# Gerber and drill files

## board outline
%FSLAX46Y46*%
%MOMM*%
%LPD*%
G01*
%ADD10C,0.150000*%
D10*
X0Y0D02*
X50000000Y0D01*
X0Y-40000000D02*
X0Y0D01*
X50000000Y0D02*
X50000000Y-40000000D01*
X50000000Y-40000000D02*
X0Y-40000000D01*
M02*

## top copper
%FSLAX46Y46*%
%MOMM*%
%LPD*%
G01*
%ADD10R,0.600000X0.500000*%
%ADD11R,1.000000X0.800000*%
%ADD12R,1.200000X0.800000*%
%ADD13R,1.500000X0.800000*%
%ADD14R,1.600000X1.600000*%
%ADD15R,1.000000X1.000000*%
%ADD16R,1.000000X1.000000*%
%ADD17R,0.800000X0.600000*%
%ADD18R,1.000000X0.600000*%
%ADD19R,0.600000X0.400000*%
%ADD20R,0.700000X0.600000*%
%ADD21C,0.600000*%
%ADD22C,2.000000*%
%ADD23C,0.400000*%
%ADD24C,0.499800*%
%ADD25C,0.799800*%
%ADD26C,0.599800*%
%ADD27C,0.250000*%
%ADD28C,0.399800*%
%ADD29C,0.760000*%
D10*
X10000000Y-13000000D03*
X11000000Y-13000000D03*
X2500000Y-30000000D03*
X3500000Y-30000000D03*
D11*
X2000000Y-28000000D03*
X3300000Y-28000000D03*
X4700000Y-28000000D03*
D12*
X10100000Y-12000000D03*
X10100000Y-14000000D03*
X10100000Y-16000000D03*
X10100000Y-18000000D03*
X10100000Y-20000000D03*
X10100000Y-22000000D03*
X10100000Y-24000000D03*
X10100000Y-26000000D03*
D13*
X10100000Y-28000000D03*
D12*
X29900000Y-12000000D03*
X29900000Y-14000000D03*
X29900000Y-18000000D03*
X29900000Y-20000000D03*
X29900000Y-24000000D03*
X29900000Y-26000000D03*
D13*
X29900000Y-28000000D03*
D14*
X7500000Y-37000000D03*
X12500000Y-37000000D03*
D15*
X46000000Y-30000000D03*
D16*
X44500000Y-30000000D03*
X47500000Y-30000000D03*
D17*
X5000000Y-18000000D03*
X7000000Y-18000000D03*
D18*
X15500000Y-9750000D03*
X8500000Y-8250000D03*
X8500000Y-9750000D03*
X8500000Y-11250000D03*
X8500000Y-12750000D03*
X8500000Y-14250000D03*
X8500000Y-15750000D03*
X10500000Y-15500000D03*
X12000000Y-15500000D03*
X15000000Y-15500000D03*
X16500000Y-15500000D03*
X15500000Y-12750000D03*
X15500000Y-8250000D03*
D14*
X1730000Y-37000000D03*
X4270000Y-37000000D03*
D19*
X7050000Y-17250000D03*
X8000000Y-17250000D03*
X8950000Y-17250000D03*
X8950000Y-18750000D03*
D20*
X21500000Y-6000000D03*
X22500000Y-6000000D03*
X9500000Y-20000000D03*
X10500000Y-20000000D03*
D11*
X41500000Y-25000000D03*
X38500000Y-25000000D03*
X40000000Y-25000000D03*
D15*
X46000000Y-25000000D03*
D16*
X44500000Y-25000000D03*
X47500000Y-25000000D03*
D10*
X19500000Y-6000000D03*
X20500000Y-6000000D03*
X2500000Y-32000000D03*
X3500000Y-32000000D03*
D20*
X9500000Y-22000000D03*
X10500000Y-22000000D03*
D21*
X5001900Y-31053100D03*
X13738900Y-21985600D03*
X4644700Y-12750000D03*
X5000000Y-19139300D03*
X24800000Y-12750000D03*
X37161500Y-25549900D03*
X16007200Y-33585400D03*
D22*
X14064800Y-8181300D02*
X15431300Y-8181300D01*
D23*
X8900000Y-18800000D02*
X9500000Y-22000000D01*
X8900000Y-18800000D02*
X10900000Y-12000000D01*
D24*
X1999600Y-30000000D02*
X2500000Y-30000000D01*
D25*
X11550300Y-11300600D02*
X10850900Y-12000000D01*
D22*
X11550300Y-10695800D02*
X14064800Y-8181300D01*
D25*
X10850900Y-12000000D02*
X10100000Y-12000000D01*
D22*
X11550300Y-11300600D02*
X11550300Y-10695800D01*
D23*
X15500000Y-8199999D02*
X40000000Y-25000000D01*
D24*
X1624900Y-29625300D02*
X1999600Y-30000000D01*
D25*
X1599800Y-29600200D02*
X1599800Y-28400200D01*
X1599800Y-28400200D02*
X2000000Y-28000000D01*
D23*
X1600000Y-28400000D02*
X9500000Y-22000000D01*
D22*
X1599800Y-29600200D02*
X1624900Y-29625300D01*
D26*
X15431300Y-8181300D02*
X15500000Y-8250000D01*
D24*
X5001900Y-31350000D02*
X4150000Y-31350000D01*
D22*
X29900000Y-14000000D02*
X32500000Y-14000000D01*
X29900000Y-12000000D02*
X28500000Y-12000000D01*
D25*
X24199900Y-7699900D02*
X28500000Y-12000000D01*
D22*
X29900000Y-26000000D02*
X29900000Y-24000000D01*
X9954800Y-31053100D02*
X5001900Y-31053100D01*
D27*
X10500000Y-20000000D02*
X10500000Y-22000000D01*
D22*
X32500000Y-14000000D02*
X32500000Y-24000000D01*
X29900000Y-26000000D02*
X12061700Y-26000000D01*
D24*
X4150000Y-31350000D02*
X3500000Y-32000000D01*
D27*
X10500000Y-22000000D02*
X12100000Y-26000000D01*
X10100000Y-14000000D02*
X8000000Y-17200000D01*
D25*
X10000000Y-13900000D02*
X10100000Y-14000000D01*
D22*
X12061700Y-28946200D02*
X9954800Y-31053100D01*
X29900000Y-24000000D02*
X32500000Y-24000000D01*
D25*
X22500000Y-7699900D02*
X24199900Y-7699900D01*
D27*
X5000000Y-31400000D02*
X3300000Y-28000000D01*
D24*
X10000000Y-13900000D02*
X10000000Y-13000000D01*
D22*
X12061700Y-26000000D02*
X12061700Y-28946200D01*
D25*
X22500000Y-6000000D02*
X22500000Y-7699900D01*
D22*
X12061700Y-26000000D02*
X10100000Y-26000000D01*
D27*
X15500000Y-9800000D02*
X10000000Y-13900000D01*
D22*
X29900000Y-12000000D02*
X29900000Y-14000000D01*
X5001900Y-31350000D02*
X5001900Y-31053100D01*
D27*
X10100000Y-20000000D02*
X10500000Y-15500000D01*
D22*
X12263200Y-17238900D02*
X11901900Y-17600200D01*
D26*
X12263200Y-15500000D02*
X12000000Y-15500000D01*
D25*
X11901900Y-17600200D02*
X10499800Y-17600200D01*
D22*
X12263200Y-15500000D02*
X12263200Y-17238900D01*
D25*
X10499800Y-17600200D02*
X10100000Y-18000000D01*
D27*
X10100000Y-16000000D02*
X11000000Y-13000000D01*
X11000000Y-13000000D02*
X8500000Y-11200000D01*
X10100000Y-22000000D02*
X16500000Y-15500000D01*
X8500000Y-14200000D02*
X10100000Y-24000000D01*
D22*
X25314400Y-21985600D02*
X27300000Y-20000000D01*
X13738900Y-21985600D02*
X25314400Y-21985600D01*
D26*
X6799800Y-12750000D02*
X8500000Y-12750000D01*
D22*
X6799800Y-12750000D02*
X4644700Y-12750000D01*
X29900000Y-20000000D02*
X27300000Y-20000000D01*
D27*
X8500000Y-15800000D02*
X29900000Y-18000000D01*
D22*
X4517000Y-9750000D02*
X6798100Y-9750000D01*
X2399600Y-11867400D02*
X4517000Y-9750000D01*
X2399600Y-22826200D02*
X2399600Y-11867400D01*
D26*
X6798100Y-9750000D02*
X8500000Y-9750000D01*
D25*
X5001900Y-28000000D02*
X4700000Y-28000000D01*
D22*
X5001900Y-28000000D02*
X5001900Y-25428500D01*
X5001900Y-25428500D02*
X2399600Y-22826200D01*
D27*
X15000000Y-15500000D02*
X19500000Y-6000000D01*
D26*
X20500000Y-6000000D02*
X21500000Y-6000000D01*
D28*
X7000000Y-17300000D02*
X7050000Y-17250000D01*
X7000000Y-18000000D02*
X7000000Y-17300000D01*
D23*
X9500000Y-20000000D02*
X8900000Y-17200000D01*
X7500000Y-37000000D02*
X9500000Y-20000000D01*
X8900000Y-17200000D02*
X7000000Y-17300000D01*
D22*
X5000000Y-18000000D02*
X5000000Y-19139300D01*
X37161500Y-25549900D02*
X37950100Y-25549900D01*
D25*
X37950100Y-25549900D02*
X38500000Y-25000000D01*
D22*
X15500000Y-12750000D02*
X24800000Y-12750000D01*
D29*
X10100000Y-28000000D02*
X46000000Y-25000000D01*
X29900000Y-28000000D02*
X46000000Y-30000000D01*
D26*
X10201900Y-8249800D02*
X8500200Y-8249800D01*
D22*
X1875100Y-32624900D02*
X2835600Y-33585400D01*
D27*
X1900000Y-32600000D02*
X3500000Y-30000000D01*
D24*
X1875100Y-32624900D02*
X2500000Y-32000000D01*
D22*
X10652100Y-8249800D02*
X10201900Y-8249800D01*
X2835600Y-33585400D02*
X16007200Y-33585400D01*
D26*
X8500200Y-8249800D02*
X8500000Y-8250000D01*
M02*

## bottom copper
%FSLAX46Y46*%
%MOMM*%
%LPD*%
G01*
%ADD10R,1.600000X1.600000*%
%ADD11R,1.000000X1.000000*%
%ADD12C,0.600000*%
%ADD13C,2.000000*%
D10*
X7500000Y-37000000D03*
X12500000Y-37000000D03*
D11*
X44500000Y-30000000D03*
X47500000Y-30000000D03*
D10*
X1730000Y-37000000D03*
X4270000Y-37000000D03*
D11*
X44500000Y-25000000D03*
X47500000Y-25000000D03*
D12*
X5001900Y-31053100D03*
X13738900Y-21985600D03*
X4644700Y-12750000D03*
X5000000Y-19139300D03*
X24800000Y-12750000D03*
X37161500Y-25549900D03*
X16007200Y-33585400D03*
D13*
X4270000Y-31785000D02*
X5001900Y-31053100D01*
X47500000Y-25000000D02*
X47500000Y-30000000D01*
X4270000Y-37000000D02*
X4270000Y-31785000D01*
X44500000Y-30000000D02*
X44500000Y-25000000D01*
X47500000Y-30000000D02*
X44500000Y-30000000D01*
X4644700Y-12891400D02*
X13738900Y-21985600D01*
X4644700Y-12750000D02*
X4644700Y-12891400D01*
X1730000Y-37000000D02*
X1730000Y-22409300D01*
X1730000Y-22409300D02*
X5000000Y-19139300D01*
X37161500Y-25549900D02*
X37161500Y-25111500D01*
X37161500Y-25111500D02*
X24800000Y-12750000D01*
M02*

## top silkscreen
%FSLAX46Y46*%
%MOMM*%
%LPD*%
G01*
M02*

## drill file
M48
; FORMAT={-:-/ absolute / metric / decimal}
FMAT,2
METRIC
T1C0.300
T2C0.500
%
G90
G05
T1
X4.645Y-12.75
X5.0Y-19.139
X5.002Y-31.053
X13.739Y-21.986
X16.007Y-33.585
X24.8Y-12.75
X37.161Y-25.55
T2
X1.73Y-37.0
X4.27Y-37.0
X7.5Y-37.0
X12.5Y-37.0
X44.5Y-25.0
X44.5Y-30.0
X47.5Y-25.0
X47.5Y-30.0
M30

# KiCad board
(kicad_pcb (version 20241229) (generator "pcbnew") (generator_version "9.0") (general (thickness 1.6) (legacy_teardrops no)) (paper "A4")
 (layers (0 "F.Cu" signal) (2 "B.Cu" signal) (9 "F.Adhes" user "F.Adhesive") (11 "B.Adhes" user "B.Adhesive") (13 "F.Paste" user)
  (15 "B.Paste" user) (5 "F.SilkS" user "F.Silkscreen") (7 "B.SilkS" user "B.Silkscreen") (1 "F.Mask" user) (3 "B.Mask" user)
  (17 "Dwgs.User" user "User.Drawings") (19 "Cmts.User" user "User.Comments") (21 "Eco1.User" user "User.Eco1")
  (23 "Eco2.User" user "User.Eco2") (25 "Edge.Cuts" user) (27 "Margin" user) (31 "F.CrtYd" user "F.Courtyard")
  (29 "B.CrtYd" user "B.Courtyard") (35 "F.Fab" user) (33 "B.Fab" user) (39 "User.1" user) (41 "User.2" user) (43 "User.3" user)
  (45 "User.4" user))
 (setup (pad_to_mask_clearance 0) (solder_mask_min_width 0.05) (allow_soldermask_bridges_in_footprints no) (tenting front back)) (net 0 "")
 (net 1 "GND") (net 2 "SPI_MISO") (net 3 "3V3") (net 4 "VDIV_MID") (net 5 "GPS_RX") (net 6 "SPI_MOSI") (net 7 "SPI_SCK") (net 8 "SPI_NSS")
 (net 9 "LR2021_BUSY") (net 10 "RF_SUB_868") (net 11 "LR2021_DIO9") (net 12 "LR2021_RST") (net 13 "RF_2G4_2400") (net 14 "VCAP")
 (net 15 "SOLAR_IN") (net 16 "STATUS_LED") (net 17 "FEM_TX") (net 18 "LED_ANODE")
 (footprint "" (layer "F.Cu") (at 10.5 13)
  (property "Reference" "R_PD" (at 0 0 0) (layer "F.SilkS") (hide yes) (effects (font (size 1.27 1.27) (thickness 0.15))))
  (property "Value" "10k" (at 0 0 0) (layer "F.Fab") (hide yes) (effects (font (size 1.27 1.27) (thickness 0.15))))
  (pad "1" smd rect (at -0.5 0) (size 0.6 0.5) (layers "F.Cu" "F.Mask") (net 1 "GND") (thermal_bridge_angle 45))
  (pad "2" smd rect (at 0.5 0) (size 0.6 0.5) (layers "F.Cu" "F.Mask") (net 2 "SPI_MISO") (thermal_bridge_angle 45)))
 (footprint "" (layer "F.Cu") (at 3 30)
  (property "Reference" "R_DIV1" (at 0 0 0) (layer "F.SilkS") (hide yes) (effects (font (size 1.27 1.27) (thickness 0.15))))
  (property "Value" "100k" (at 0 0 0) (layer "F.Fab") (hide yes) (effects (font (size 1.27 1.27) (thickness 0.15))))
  (pad "1" smd rect (at -0.5 0) (size 0.6 0.5) (layers "F.Cu" "F.Mask") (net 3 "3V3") (thermal_bridge_angle 45))
  (pad "2" smd rect (at 0.5 0) (size 0.6 0.5) (layers "F.Cu" "F.Mask") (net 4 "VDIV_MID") (thermal_bridge_angle 45)))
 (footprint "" (layer "F.Cu") (at 4 28)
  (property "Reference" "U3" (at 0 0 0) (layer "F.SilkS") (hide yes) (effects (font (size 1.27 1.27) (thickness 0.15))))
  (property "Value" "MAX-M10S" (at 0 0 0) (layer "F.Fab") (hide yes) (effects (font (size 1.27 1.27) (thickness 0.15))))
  (pad "1" smd rect (at -2 0) (size 1 0.8) (layers "F.Cu" "F.Mask") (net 3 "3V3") (thermal_bridge_angle 45))
  (pad "2" smd rect (at -0.7 0) (size 1 0.8) (layers "F.Cu" "F.Mask") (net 1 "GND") (thermal_bridge_angle 45))
  (pad "3" smd rect (at 0.7 0) (size 1 0.8) (layers "F.Cu" "F.Mask") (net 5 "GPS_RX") (thermal_bridge_angle 45)))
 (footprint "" (layer "F.Cu") (at 20 20)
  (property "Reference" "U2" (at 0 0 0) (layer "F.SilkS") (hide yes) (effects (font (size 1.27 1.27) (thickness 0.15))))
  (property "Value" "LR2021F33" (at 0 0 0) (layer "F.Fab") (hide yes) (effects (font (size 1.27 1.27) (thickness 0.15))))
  (pad "1" smd rect (at -9.9 -8) (size 1.2 0.8) (layers "F.Cu" "F.Mask") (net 3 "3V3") (thermal_bridge_angle 45))
  (pad "2" smd rect (at -9.9 -6) (size 1.2 0.8) (layers "F.Cu" "F.Mask") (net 1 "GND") (thermal_bridge_angle 45))
  (pad "3" smd rect (at -9.9 -4) (size 1.2 0.8) (layers "F.Cu" "F.Mask") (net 2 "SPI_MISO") (thermal_bridge_angle 45))
  (pad "4" smd rect (at -9.9 -2) (size 1.2 0.8) (layers "F.Cu" "F.Mask") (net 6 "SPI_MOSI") (thermal_bridge_angle 45))
  (pad "5" smd rect (at -9.9 0) (size 1.2 0.8) (layers "F.Cu" "F.Mask") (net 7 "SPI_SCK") (thermal_bridge_angle 45))
  (pad "6" smd rect (at -9.9 2) (size 1.2 0.8) (layers "F.Cu" "F.Mask") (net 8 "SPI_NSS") (thermal_bridge_angle 45))
  (pad "7" smd rect (at -9.9 4) (size 1.2 0.8) (layers "F.Cu" "F.Mask") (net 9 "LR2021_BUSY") (thermal_bridge_angle 45))
  (pad "8" smd rect (at -9.9 6) (size 1.2 0.8) (layers "F.Cu" "F.Mask") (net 1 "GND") (thermal_bridge_angle 45))
  (pad "9" smd rect (at -9.9 8) (size 1.5 0.8) (layers "F.Cu" "F.Mask") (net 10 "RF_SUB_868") (thermal_bridge_angle 45))
  (pad "10" smd rect (at 9.9 -8) (size 1.2 0.8) (layers "F.Cu" "F.Mask") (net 1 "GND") (thermal_bridge_angle 45))
  (pad "11" smd rect (at 9.9 -6) (size 1.2 0.8) (layers "F.Cu" "F.Mask") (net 1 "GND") (thermal_bridge_angle 45))
  (pad "13" smd rect (at 9.9 -2) (size 1.2 0.8) (layers "F.Cu" "F.Mask") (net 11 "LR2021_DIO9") (thermal_bridge_angle 45))
  (pad "14" smd rect (at 9.9 0) (size 1.2 0.8) (layers "F.Cu" "F.Mask") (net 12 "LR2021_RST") (thermal_bridge_angle 45))
  (pad "16" smd rect (at 9.9 4) (size 1.2 0.8) (layers "F.Cu" "F.Mask") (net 1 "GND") (thermal_bridge_angle 45))
  (pad "17" smd rect (at 9.9 6) (size 1.2 0.8) (layers "F.Cu" "F.Mask") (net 1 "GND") (thermal_bridge_angle 45))
  (pad "18" smd rect (at 9.9 8) (size 1.5 0.8) (layers "F.Cu" "F.Mask") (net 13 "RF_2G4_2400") (thermal_bridge_angle 45)))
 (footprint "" (layer "F.Cu") (at 10 37)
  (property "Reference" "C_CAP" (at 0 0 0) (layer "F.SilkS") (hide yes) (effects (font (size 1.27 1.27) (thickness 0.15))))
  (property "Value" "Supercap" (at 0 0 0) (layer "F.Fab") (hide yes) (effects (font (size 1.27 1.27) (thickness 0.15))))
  (pad "1" thru_hole rect (at -2.5 0) (size 1.6 1.6) (drill 0.5) (layers "*.Cu" "*.Mask") (remove_unused_layers no) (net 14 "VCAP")
   (thermal_bridge_angle 45))
  (pad "2" thru_hole rect (at 2.5 0) (size 1.6 1.6) (drill 0.5) (layers "*.Cu" "*.Mask") (remove_unused_layers no) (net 1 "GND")
   (thermal_bridge_angle 45)))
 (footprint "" (layer "F.Cu") (at 46 30)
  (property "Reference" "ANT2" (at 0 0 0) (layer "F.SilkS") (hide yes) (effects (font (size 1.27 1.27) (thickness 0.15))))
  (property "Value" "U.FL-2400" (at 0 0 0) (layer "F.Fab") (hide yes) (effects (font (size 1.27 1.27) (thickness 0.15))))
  (pad "1" smd rect (at 0 0) (size 1 1) (layers "F.Cu" "F.Mask") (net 13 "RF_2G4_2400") (thermal_bridge_angle 45))
  (pad "2" thru_hole rect (at -1.5 0) (size 1 1) (drill 0.5) (layers "*.Cu" "*.Mask") (remove_unused_layers no) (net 1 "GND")
   (thermal_bridge_angle 45))
  (pad "3" thru_hole rect (at 1.5 0) (size 1 1) (drill 0.5) (layers "*.Cu" "*.Mask") (remove_unused_layers no) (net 1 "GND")
   (thermal_bridge_angle 45)))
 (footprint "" (layer "F.Cu") (at 6 18)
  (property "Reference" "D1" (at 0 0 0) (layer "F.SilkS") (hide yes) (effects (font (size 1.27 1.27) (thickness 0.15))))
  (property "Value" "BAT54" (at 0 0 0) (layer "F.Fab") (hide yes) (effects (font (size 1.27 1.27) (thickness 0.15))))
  (pad "A" smd rect (at -1 0) (size 0.8 0.6) (layers "F.Cu" "F.Mask") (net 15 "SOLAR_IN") (thermal_bridge_angle 45))
  (pad "K" smd rect (at 1 0) (size 0.8 0.6) (layers "F.Cu" "F.Mask") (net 14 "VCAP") (thermal_bridge_angle 45)))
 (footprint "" (layer "F.Cu") (at 12 12)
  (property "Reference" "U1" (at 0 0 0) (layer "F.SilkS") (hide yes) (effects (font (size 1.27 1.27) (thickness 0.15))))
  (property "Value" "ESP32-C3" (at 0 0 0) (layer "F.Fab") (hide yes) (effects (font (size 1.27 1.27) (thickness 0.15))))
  (pad "GND" smd rect (at 3.5 -2.25) (size 1 0.6) (layers "F.Cu" "F.Mask") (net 1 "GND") (thermal_bridge_angle 45))
  (pad "GPIO0" smd rect (at -3.5 -3.75) (size 1 0.6) (layers "F.Cu" "F.Mask") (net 4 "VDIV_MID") (thermal_bridge_angle 45))
  (pad "GPIO1" smd rect (at -3.5 -2.25) (size 1 0.6) (layers "F.Cu" "F.Mask") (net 5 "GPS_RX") (thermal_bridge_angle 45))
  (pad "GPIO2" smd rect (at -3.5 -0.75) (size 1 0.6) (layers "F.Cu" "F.Mask") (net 2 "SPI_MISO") (thermal_bridge_angle 45))
  (pad "GPIO3" smd rect (at -3.5 0.75) (size 1 0.6) (layers "F.Cu" "F.Mask") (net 12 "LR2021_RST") (thermal_bridge_angle 45))
  (pad "GPIO4" smd rect (at -3.5 2.25) (size 1 0.6) (layers "F.Cu" "F.Mask") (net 9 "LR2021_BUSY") (thermal_bridge_angle 45))
  (pad "GPIO5" smd rect (at -3.5 3.75) (size 1 0.6) (layers "F.Cu" "F.Mask") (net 11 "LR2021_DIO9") (thermal_bridge_angle 45))
  (pad "GPIO6" smd rect (at -1.5 3.5) (size 1 0.6) (layers "F.Cu" "F.Mask") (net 7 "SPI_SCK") (thermal_bridge_angle 45))
  (pad "GPIO7" smd rect (at 0 3.5) (size 1 0.6) (layers "F.Cu" "F.Mask") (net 6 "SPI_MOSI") (thermal_bridge_angle 45))
  (pad "GPIO9" smd rect (at 3 3.5) (size 1 0.6) (layers "F.Cu" "F.Mask") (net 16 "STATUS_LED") (thermal_bridge_angle 45))
  (pad "GPIO10" smd rect (at 4.5 3.5) (size 1 0.6) (layers "F.Cu" "F.Mask") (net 8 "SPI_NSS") (thermal_bridge_angle 45))
  (pad "GPIO19" smd rect (at 3.5 0.75) (size 1 0.6) (layers "F.Cu" "F.Mask") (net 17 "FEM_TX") (thermal_bridge_angle 45))
  (pad "VCC" smd rect (at 3.5 -3.75) (size 1 0.6) (layers "F.Cu" "F.Mask") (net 3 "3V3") (thermal_bridge_angle 45)))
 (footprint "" (layer "F.Cu") (at 3 37)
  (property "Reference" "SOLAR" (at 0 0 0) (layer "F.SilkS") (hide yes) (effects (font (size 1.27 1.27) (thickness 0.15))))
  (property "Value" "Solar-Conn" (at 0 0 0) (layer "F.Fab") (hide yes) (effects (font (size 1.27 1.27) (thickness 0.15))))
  (pad "1" thru_hole rect (at -1.27 0) (size 1.6 1.6) (drill 0.5) (layers "*.Cu" "*.Mask") (remove_unused_layers no) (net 15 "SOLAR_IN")
   (thermal_bridge_angle 45))
  (pad "2" thru_hole rect (at 1.27 0) (size 1.6 1.6) (drill 0.5) (layers "*.Cu" "*.Mask") (remove_unused_layers no) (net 1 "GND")
   (thermal_bridge_angle 45)))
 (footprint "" (layer "F.Cu") (at 8 18)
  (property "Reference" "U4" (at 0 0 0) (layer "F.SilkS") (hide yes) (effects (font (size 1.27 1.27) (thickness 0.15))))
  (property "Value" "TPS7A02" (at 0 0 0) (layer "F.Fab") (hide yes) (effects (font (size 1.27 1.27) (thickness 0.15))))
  (pad "1" smd rect (at -0.95 -0.75) (size 0.6 0.4) (layers "F.Cu" "F.Mask") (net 14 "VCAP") (thermal_bridge_angle 45))
  (pad "2" smd rect (at 0 -0.75) (size 0.6 0.4) (layers "F.Cu" "F.Mask") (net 1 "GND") (thermal_bridge_angle 45))
  (pad "3" smd rect (at 0.95 -0.75) (size 0.6 0.4) (layers "F.Cu" "F.Mask") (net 14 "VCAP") (thermal_bridge_angle 45))
  (pad "4" smd rect (at 0.95 0.75) (size 0.6 0.4) (layers "F.Cu" "F.Mask") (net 3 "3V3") (thermal_bridge_angle 45)))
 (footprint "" (layer "F.Cu") (at 22 6)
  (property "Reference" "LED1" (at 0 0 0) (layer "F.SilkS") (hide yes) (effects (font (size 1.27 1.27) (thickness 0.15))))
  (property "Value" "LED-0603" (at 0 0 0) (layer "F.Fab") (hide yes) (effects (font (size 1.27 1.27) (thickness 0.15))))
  (pad "A" smd rect (at -0.5 0) (size 0.7 0.6) (layers "F.Cu" "F.Mask") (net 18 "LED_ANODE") (thermal_bridge_angle 45))
  (pad "K" smd rect (at 0.5 0) (size 0.7 0.6) (layers "F.Cu" "F.Mask") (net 1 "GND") (thermal_bridge_angle 45)))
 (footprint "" (layer "F.Cu") (at 10 20)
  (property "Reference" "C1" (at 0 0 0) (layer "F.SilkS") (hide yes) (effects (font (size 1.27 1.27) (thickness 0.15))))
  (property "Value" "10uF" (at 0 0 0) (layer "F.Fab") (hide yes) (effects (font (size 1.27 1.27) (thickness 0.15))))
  (pad "1" smd rect (at -0.5 0) (size 0.7 0.6) (layers "F.Cu" "F.Mask") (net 14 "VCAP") (thermal_bridge_angle 45))
  (pad "2" smd rect (at 0.5 0) (size 0.7 0.6) (layers "F.Cu" "F.Mask") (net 1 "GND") (thermal_bridge_angle 45)))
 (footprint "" (layer "F.Cu") (at 40 25)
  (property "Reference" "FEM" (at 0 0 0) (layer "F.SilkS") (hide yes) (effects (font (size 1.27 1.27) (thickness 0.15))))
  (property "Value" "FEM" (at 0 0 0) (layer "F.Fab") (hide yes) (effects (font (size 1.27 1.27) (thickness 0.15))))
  (pad "GND" smd rect (at 1.5 0) (size 1 0.8) (layers "F.Cu" "F.Mask") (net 1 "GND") (thermal_bridge_angle 45))
  (pad "TX" smd rect (at -1.5 0) (size 1 0.8) (layers "F.Cu" "F.Mask") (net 17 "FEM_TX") (thermal_bridge_angle 45))
  (pad "VCC" smd rect (at 0 0) (size 1 0.8) (layers "F.Cu" "F.Mask") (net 3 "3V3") (thermal_bridge_angle 45)))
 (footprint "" (layer "F.Cu") (at 46 25)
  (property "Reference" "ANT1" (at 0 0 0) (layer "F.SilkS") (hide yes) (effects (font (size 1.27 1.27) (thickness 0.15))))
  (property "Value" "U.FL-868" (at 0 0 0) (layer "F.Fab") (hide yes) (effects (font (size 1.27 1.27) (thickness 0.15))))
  (pad "1" smd rect (at 0 0) (size 1 1) (layers "F.Cu" "F.Mask") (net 10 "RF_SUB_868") (thermal_bridge_angle 45))
  (pad "2" thru_hole rect (at -1.5 0) (size 1 1) (drill 0.5) (layers "*.Cu" "*.Mask") (remove_unused_layers no) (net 1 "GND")
   (thermal_bridge_angle 45))
  (pad "3" thru_hole rect (at 1.5 0) (size 1 1) (drill 0.5) (layers "*.Cu" "*.Mask") (remove_unused_layers no) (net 1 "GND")
   (thermal_bridge_angle 45)))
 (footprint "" (layer "F.Cu") (at 20 6)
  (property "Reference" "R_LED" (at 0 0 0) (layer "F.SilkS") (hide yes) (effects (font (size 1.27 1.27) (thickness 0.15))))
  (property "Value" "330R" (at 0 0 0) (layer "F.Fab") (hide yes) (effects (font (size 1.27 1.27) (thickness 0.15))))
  (pad "1" smd rect (at -0.5 0) (size 0.6 0.5) (layers "F.Cu" "F.Mask") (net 16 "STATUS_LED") (thermal_bridge_angle 45))
  (pad "2" smd rect (at 0.5 0) (size 0.6 0.5) (layers "F.Cu" "F.Mask") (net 18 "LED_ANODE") (thermal_bridge_angle 45)))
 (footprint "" (layer "F.Cu") (at 3 32)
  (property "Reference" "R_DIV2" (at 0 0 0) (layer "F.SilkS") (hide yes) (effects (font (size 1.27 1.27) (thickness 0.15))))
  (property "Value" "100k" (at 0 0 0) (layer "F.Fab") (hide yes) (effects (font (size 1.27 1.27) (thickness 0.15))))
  (pad "1" smd rect (at -0.5 0) (size 0.6 0.5) (layers "F.Cu" "F.Mask") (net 4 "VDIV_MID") (thermal_bridge_angle 45))
  (pad "2" smd rect (at 0.5 0) (size 0.6 0.5) (layers "F.Cu" "F.Mask") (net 1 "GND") (thermal_bridge_angle 45)))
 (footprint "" (layer "F.Cu") (at 10 22)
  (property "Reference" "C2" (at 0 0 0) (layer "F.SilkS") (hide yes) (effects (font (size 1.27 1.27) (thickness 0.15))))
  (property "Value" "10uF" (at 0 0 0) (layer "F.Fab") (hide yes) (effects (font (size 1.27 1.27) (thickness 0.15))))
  (pad "1" smd rect (at -0.5 0) (size 0.7 0.6) (layers "F.Cu" "F.Mask") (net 3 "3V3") (thermal_bridge_angle 45))
  (pad "2" smd rect (at 0.5 0) (size 0.7 0.6) (layers "F.Cu" "F.Mask") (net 1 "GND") (thermal_bridge_angle 45)))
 (gr_line (start 0 0) (end 50 0) (stroke (width 0.15) (type default)) (layer "Edge.Cuts"))
 (gr_line (start 0 40) (end 0 0) (stroke (width 0.15) (type default)) (layer "Edge.Cuts"))
 (gr_line (start 50 0) (end 50 40) (stroke (width 0.15) (type default)) (layer "Edge.Cuts"))
 (gr_line (start 50 40) (end 0 40) (stroke (width 0.15) (type default)) (layer "Edge.Cuts"))
 (segment (start 14.0648 8.1813) (end 15.4313 8.1813) (width 2) (layer "F.Cu") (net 3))
 (segment (start 8.9 18.8) (end 9.5 22) (width 0.4) (layer "F.Cu") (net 3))
 (segment (start 8.9 18.8) (end 10.9 12) (width 0.4) (layer "F.Cu") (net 3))
 (segment (start 1.9996 30) (end 2.5 30) (width 0.4998) (layer "F.Cu") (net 3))
 (segment (start 11.5503 11.3006) (end 10.8509 12) (width 0.7998) (layer "F.Cu") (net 3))
 (segment (start 11.5503 10.6958) (end 14.0648 8.1813) (width 2) (layer "F.Cu") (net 3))
 (segment (start 10.8509 12) (end 10.1 12) (width 0.7998) (layer "F.Cu") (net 3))
 (segment (start 11.5503 11.3006) (end 11.5503 10.6958) (width 2) (layer "F.Cu") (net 3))
 (segment (start 15.5 8.199999) (end 40 25) (width 0.4) (layer "F.Cu") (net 3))
 (segment (start 1.6249 29.6253) (end 1.9996 30) (width 0.4998) (layer "F.Cu") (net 3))
 (segment (start 1.5998 29.6002) (end 1.5998 28.4002) (width 0.7998) (layer "F.Cu") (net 3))
 (segment (start 1.5998 28.4002) (end 2 28) (width 0.7998) (layer "F.Cu") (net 3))
 (segment (start 1.6 28.4) (end 9.5 22) (width 0.4) (layer "F.Cu") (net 3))
 (segment (start 1.5998 29.6002) (end 1.6249 29.6253) (width 2) (layer "F.Cu") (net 3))
 (segment (start 15.4313 8.1813) (end 15.5 8.25) (width 0.5998) (layer "F.Cu") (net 3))
 (segment (start 5.0019 31.35) (end 4.15 31.35) (width 0.4998) (layer "F.Cu") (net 1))
 (segment (start 29.9 14) (end 32.5 14) (width 2) (layer "F.Cu") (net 1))
 (segment (start 29.9 12) (end 28.5 12) (width 2) (layer "F.Cu") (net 1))
 (segment (start 24.1999 7.6999) (end 28.5 12) (width 0.7998) (layer "F.Cu") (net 1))
 (segment (start 29.9 26) (end 29.9 24) (width 2) (layer "F.Cu") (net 1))
 (segment (start 9.9548 31.0531) (end 5.0019 31.0531) (width 2) (layer "F.Cu") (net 1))
 (segment (start 10.5 20) (end 10.5 22) (width 0.25) (layer "F.Cu") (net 1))
 (segment (start 32.5 14) (end 32.5 24) (width 2) (layer "F.Cu") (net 1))
 (segment (start 29.9 26) (end 12.0617 26) (width 2) (layer "F.Cu") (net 1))
 (segment (start 4.15 31.35) (end 3.5 32) (width 0.4998) (layer "F.Cu") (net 1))
 (segment (start 10.5 22) (end 12.1 26) (width 0.25) (layer "F.Cu") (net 1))
 (segment (start 10.1 14) (end 8 17.2) (width 0.25) (layer "F.Cu") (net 1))
 (segment (start 10 13.9) (end 10.1 14) (width 0.7998) (layer "F.Cu") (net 1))
 (segment (start 12.0617 28.9462) (end 9.9548 31.0531) (width 2) (layer "F.Cu") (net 1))
 (segment (start 29.9 24) (end 32.5 24) (width 2) (layer "F.Cu") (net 1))
 (segment (start 22.5 7.6999) (end 24.1999 7.6999) (width 0.7998) (layer "F.Cu") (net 1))
 (segment (start 5 31.4) (end 3.3 28) (width 0.25) (layer "F.Cu") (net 1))
 (segment (start 10 13.9) (end 10 13) (width 0.4998) (layer "F.Cu") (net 1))
 (segment (start 12.0617 26) (end 12.0617 28.9462) (width 2) (layer "F.Cu") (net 1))
 (segment (start 22.5 6) (end 22.5 7.6999) (width 0.7998) (layer "F.Cu") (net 1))
 (segment (start 12.0617 26) (end 10.1 26) (width 2) (layer "F.Cu") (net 1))
 (segment (start 15.5 9.8) (end 10 13.9) (width 0.25) (layer "F.Cu") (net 1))
 (segment (start 29.9 12) (end 29.9 14) (width 2) (layer "F.Cu") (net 1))
 (segment (start 5.0019 31.35) (end 5.0019 31.0531) (width 2) (layer "F.Cu") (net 1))
 (via (at 5.0019 31.0531) (size 0.6) (drill 0.3) (layers "F.Cu" "B.Cu") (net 1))
 (segment (start 4.27 31.785) (end 5.0019 31.0531) (width 2) (layer "B.Cu") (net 1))
 (segment (start 47.5 25) (end 47.5 30) (width 2) (layer "B.Cu") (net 1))
 (segment (start 4.27 37) (end 4.27 31.785) (width 2) (layer "B.Cu") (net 1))
 (segment (start 44.5 30) (end 44.5 25) (width 2) (layer "B.Cu") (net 1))
 (segment (start 47.5 30) (end 44.5 30) (width 2) (layer "B.Cu") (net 1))
 (segment (start 10.1 20) (end 10.5 15.5) (width 0.25) (layer "F.Cu") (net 7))
 (segment (start 12.2632 17.2389) (end 11.9019 17.6002) (width 2) (layer "F.Cu") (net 6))
 (segment (start 12.2632 15.5) (end 12 15.5) (width 0.5998) (layer "F.Cu") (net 6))
 (segment (start 11.9019 17.6002) (end 10.4998 17.6002) (width 0.7998) (layer "F.Cu") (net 6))
 (segment (start 12.2632 15.5) (end 12.2632 17.2389) (width 2) (layer "F.Cu") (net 6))
 (segment (start 10.4998 17.6002) (end 10.1 18) (width 0.7998) (layer "F.Cu") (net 6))
 (segment (start 10.1 16) (end 11 13) (width 0.25) (layer "F.Cu") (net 2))
 (segment (start 11 13) (end 8.5 11.2) (width 0.25) (layer "F.Cu") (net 2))
 (segment (start 10.1 22) (end 16.5 15.5) (width 0.25) (layer "F.Cu") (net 8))
 (segment (start 8.5 14.2) (end 10.1 24) (width 0.25) (layer "F.Cu") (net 9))
 (segment (start 25.3144 21.9856) (end 27.3 20) (width 2) (layer "F.Cu") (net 12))
 (segment (start 13.7389 21.9856) (end 25.3144 21.9856) (width 2) (layer "F.Cu") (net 12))
 (segment (start 6.7998 12.75) (end 8.5 12.75) (width 0.5998) (layer "F.Cu") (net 12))
 (segment (start 6.7998 12.75) (end 4.6447 12.75) (width 2) (layer "F.Cu") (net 12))
 (segment (start 29.9 20) (end 27.3 20) (width 2) (layer "F.Cu") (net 12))
 (via (at 13.7389 21.9856) (size 0.6) (drill 0.3) (layers "F.Cu" "B.Cu") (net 12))
 (via (at 4.6447 12.75) (size 0.6) (drill 0.3) (layers "F.Cu" "B.Cu") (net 12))
 (segment (start 4.6447 12.8914) (end 13.7389 21.9856) (width 2) (layer "B.Cu") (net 12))
 (segment (start 4.6447 12.75) (end 4.6447 12.8914) (width 2) (layer "B.Cu") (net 12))
 (segment (start 8.5 15.8) (end 29.9 18) (width 0.25) (layer "F.Cu") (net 11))
 (segment (start 4.517 9.75) (end 6.7981 9.75) (width 2) (layer "F.Cu") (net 5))
 (segment (start 2.3996 11.8674) (end 4.517 9.75) (width 2) (layer "F.Cu") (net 5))
 (segment (start 2.3996 22.8262) (end 2.3996 11.8674) (width 2) (layer "F.Cu") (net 5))
 (segment (start 6.7981 9.75) (end 8.5 9.75) (width 0.5998) (layer "F.Cu") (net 5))
 (segment (start 5.0019 28) (end 4.7 28) (width 0.7998) (layer "F.Cu") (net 5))
 (segment (start 5.0019 28) (end 5.0019 25.4285) (width 2) (layer "F.Cu") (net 5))
 (segment (start 5.0019 25.4285) (end 2.3996 22.8262) (width 2) (layer "F.Cu") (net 5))
 (segment (start 15 15.5) (end 19.5 6) (width 0.25) (layer "F.Cu") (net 16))
 (segment (start 20.5 6) (end 21.5 6) (width 0.5998) (layer "F.Cu") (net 18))
 (segment (start 7 17.3) (end 7.05 17.25) (width 0.3998) (layer "F.Cu") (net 14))
 (segment (start 7 18) (end 7 17.3) (width 0.3998) (layer "F.Cu") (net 14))
 (segment (start 9.5 20) (end 8.9 17.2) (width 0.4) (layer "F.Cu") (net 14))
 (segment (start 7.5 37) (end 9.5 20) (width 0.4) (layer "F.Cu") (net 14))
 (segment (start 8.9 17.2) (end 7 17.3) (width 0.4) (layer "F.Cu") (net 14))
 (segment (start 5 18) (end 5 19.1393) (width 2) (layer "F.Cu") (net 15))
 (via (at 5 19.1393) (size 0.6) (drill 0.3) (layers "F.Cu" "B.Cu") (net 15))
 (segment (start 1.73 37) (end 1.73 22.4093) (width 2) (layer "B.Cu") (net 15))
 (segment (start 1.73 22.4093) (end 5 19.1393) (width 2) (layer "B.Cu") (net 15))
 (segment (start 37.1615 25.5499) (end 37.9501 25.5499) (width 2) (layer "F.Cu") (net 17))
 (segment (start 37.9501 25.5499) (end 38.5 25) (width 0.7998) (layer "F.Cu") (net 17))
 (segment (start 15.5 12.75) (end 24.8 12.75) (width 2) (layer "F.Cu") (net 17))
 (via (at 24.8 12.75) (size 0.6) (drill 0.3) (layers "F.Cu" "B.Cu") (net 17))
 (via (at 37.1615 25.5499) (size 0.6) (drill 0.3) (layers "F.Cu" "B.Cu") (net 17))
 (segment (start 37.1615 25.5499) (end 37.1615 25.1115) (width 2) (layer "B.Cu") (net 17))
 (segment (start 37.1615 25.1115) (end 24.8 12.75) (width 2) (layer "B.Cu") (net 17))
 (segment (start 10.1 28) (end 46 25) (width 0.76) (layer "F.Cu") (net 10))
 (segment (start 29.9 28) (end 46 30) (width 0.76) (layer "F.Cu") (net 13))
 (segment (start 10.2019 8.2498) (end 8.5002 8.2498) (width 0.5998) (layer "F.Cu") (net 4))
 (segment (start 1.8751 32.6249) (end 2.8356 33.5854) (width 2) (layer "F.Cu") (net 4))
 (segment (start 1.9 32.6) (end 3.5 30) (width 0.25) (layer "F.Cu") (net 4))
 (segment (start 1.8751 32.6249) (end 2.5 32) (width 0.4998) (layer "F.Cu") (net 4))
 (segment (start 10.6521 8.2498) (end 10.2019 8.2498) (width 2) (layer "F.Cu") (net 4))
 (segment (start 2.8356 33.5854) (end 16.0072 33.5854) (width 2) (layer "F.Cu") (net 4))
 (segment (start 8.5002 8.2498) (end 8.5 8.25) (width 0.5998) (layer "F.Cu") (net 4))
 (via (at 16.0072 33.5854) (size 0.6) (drill 0.3) (layers "F.Cu" "B.Cu") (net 4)))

